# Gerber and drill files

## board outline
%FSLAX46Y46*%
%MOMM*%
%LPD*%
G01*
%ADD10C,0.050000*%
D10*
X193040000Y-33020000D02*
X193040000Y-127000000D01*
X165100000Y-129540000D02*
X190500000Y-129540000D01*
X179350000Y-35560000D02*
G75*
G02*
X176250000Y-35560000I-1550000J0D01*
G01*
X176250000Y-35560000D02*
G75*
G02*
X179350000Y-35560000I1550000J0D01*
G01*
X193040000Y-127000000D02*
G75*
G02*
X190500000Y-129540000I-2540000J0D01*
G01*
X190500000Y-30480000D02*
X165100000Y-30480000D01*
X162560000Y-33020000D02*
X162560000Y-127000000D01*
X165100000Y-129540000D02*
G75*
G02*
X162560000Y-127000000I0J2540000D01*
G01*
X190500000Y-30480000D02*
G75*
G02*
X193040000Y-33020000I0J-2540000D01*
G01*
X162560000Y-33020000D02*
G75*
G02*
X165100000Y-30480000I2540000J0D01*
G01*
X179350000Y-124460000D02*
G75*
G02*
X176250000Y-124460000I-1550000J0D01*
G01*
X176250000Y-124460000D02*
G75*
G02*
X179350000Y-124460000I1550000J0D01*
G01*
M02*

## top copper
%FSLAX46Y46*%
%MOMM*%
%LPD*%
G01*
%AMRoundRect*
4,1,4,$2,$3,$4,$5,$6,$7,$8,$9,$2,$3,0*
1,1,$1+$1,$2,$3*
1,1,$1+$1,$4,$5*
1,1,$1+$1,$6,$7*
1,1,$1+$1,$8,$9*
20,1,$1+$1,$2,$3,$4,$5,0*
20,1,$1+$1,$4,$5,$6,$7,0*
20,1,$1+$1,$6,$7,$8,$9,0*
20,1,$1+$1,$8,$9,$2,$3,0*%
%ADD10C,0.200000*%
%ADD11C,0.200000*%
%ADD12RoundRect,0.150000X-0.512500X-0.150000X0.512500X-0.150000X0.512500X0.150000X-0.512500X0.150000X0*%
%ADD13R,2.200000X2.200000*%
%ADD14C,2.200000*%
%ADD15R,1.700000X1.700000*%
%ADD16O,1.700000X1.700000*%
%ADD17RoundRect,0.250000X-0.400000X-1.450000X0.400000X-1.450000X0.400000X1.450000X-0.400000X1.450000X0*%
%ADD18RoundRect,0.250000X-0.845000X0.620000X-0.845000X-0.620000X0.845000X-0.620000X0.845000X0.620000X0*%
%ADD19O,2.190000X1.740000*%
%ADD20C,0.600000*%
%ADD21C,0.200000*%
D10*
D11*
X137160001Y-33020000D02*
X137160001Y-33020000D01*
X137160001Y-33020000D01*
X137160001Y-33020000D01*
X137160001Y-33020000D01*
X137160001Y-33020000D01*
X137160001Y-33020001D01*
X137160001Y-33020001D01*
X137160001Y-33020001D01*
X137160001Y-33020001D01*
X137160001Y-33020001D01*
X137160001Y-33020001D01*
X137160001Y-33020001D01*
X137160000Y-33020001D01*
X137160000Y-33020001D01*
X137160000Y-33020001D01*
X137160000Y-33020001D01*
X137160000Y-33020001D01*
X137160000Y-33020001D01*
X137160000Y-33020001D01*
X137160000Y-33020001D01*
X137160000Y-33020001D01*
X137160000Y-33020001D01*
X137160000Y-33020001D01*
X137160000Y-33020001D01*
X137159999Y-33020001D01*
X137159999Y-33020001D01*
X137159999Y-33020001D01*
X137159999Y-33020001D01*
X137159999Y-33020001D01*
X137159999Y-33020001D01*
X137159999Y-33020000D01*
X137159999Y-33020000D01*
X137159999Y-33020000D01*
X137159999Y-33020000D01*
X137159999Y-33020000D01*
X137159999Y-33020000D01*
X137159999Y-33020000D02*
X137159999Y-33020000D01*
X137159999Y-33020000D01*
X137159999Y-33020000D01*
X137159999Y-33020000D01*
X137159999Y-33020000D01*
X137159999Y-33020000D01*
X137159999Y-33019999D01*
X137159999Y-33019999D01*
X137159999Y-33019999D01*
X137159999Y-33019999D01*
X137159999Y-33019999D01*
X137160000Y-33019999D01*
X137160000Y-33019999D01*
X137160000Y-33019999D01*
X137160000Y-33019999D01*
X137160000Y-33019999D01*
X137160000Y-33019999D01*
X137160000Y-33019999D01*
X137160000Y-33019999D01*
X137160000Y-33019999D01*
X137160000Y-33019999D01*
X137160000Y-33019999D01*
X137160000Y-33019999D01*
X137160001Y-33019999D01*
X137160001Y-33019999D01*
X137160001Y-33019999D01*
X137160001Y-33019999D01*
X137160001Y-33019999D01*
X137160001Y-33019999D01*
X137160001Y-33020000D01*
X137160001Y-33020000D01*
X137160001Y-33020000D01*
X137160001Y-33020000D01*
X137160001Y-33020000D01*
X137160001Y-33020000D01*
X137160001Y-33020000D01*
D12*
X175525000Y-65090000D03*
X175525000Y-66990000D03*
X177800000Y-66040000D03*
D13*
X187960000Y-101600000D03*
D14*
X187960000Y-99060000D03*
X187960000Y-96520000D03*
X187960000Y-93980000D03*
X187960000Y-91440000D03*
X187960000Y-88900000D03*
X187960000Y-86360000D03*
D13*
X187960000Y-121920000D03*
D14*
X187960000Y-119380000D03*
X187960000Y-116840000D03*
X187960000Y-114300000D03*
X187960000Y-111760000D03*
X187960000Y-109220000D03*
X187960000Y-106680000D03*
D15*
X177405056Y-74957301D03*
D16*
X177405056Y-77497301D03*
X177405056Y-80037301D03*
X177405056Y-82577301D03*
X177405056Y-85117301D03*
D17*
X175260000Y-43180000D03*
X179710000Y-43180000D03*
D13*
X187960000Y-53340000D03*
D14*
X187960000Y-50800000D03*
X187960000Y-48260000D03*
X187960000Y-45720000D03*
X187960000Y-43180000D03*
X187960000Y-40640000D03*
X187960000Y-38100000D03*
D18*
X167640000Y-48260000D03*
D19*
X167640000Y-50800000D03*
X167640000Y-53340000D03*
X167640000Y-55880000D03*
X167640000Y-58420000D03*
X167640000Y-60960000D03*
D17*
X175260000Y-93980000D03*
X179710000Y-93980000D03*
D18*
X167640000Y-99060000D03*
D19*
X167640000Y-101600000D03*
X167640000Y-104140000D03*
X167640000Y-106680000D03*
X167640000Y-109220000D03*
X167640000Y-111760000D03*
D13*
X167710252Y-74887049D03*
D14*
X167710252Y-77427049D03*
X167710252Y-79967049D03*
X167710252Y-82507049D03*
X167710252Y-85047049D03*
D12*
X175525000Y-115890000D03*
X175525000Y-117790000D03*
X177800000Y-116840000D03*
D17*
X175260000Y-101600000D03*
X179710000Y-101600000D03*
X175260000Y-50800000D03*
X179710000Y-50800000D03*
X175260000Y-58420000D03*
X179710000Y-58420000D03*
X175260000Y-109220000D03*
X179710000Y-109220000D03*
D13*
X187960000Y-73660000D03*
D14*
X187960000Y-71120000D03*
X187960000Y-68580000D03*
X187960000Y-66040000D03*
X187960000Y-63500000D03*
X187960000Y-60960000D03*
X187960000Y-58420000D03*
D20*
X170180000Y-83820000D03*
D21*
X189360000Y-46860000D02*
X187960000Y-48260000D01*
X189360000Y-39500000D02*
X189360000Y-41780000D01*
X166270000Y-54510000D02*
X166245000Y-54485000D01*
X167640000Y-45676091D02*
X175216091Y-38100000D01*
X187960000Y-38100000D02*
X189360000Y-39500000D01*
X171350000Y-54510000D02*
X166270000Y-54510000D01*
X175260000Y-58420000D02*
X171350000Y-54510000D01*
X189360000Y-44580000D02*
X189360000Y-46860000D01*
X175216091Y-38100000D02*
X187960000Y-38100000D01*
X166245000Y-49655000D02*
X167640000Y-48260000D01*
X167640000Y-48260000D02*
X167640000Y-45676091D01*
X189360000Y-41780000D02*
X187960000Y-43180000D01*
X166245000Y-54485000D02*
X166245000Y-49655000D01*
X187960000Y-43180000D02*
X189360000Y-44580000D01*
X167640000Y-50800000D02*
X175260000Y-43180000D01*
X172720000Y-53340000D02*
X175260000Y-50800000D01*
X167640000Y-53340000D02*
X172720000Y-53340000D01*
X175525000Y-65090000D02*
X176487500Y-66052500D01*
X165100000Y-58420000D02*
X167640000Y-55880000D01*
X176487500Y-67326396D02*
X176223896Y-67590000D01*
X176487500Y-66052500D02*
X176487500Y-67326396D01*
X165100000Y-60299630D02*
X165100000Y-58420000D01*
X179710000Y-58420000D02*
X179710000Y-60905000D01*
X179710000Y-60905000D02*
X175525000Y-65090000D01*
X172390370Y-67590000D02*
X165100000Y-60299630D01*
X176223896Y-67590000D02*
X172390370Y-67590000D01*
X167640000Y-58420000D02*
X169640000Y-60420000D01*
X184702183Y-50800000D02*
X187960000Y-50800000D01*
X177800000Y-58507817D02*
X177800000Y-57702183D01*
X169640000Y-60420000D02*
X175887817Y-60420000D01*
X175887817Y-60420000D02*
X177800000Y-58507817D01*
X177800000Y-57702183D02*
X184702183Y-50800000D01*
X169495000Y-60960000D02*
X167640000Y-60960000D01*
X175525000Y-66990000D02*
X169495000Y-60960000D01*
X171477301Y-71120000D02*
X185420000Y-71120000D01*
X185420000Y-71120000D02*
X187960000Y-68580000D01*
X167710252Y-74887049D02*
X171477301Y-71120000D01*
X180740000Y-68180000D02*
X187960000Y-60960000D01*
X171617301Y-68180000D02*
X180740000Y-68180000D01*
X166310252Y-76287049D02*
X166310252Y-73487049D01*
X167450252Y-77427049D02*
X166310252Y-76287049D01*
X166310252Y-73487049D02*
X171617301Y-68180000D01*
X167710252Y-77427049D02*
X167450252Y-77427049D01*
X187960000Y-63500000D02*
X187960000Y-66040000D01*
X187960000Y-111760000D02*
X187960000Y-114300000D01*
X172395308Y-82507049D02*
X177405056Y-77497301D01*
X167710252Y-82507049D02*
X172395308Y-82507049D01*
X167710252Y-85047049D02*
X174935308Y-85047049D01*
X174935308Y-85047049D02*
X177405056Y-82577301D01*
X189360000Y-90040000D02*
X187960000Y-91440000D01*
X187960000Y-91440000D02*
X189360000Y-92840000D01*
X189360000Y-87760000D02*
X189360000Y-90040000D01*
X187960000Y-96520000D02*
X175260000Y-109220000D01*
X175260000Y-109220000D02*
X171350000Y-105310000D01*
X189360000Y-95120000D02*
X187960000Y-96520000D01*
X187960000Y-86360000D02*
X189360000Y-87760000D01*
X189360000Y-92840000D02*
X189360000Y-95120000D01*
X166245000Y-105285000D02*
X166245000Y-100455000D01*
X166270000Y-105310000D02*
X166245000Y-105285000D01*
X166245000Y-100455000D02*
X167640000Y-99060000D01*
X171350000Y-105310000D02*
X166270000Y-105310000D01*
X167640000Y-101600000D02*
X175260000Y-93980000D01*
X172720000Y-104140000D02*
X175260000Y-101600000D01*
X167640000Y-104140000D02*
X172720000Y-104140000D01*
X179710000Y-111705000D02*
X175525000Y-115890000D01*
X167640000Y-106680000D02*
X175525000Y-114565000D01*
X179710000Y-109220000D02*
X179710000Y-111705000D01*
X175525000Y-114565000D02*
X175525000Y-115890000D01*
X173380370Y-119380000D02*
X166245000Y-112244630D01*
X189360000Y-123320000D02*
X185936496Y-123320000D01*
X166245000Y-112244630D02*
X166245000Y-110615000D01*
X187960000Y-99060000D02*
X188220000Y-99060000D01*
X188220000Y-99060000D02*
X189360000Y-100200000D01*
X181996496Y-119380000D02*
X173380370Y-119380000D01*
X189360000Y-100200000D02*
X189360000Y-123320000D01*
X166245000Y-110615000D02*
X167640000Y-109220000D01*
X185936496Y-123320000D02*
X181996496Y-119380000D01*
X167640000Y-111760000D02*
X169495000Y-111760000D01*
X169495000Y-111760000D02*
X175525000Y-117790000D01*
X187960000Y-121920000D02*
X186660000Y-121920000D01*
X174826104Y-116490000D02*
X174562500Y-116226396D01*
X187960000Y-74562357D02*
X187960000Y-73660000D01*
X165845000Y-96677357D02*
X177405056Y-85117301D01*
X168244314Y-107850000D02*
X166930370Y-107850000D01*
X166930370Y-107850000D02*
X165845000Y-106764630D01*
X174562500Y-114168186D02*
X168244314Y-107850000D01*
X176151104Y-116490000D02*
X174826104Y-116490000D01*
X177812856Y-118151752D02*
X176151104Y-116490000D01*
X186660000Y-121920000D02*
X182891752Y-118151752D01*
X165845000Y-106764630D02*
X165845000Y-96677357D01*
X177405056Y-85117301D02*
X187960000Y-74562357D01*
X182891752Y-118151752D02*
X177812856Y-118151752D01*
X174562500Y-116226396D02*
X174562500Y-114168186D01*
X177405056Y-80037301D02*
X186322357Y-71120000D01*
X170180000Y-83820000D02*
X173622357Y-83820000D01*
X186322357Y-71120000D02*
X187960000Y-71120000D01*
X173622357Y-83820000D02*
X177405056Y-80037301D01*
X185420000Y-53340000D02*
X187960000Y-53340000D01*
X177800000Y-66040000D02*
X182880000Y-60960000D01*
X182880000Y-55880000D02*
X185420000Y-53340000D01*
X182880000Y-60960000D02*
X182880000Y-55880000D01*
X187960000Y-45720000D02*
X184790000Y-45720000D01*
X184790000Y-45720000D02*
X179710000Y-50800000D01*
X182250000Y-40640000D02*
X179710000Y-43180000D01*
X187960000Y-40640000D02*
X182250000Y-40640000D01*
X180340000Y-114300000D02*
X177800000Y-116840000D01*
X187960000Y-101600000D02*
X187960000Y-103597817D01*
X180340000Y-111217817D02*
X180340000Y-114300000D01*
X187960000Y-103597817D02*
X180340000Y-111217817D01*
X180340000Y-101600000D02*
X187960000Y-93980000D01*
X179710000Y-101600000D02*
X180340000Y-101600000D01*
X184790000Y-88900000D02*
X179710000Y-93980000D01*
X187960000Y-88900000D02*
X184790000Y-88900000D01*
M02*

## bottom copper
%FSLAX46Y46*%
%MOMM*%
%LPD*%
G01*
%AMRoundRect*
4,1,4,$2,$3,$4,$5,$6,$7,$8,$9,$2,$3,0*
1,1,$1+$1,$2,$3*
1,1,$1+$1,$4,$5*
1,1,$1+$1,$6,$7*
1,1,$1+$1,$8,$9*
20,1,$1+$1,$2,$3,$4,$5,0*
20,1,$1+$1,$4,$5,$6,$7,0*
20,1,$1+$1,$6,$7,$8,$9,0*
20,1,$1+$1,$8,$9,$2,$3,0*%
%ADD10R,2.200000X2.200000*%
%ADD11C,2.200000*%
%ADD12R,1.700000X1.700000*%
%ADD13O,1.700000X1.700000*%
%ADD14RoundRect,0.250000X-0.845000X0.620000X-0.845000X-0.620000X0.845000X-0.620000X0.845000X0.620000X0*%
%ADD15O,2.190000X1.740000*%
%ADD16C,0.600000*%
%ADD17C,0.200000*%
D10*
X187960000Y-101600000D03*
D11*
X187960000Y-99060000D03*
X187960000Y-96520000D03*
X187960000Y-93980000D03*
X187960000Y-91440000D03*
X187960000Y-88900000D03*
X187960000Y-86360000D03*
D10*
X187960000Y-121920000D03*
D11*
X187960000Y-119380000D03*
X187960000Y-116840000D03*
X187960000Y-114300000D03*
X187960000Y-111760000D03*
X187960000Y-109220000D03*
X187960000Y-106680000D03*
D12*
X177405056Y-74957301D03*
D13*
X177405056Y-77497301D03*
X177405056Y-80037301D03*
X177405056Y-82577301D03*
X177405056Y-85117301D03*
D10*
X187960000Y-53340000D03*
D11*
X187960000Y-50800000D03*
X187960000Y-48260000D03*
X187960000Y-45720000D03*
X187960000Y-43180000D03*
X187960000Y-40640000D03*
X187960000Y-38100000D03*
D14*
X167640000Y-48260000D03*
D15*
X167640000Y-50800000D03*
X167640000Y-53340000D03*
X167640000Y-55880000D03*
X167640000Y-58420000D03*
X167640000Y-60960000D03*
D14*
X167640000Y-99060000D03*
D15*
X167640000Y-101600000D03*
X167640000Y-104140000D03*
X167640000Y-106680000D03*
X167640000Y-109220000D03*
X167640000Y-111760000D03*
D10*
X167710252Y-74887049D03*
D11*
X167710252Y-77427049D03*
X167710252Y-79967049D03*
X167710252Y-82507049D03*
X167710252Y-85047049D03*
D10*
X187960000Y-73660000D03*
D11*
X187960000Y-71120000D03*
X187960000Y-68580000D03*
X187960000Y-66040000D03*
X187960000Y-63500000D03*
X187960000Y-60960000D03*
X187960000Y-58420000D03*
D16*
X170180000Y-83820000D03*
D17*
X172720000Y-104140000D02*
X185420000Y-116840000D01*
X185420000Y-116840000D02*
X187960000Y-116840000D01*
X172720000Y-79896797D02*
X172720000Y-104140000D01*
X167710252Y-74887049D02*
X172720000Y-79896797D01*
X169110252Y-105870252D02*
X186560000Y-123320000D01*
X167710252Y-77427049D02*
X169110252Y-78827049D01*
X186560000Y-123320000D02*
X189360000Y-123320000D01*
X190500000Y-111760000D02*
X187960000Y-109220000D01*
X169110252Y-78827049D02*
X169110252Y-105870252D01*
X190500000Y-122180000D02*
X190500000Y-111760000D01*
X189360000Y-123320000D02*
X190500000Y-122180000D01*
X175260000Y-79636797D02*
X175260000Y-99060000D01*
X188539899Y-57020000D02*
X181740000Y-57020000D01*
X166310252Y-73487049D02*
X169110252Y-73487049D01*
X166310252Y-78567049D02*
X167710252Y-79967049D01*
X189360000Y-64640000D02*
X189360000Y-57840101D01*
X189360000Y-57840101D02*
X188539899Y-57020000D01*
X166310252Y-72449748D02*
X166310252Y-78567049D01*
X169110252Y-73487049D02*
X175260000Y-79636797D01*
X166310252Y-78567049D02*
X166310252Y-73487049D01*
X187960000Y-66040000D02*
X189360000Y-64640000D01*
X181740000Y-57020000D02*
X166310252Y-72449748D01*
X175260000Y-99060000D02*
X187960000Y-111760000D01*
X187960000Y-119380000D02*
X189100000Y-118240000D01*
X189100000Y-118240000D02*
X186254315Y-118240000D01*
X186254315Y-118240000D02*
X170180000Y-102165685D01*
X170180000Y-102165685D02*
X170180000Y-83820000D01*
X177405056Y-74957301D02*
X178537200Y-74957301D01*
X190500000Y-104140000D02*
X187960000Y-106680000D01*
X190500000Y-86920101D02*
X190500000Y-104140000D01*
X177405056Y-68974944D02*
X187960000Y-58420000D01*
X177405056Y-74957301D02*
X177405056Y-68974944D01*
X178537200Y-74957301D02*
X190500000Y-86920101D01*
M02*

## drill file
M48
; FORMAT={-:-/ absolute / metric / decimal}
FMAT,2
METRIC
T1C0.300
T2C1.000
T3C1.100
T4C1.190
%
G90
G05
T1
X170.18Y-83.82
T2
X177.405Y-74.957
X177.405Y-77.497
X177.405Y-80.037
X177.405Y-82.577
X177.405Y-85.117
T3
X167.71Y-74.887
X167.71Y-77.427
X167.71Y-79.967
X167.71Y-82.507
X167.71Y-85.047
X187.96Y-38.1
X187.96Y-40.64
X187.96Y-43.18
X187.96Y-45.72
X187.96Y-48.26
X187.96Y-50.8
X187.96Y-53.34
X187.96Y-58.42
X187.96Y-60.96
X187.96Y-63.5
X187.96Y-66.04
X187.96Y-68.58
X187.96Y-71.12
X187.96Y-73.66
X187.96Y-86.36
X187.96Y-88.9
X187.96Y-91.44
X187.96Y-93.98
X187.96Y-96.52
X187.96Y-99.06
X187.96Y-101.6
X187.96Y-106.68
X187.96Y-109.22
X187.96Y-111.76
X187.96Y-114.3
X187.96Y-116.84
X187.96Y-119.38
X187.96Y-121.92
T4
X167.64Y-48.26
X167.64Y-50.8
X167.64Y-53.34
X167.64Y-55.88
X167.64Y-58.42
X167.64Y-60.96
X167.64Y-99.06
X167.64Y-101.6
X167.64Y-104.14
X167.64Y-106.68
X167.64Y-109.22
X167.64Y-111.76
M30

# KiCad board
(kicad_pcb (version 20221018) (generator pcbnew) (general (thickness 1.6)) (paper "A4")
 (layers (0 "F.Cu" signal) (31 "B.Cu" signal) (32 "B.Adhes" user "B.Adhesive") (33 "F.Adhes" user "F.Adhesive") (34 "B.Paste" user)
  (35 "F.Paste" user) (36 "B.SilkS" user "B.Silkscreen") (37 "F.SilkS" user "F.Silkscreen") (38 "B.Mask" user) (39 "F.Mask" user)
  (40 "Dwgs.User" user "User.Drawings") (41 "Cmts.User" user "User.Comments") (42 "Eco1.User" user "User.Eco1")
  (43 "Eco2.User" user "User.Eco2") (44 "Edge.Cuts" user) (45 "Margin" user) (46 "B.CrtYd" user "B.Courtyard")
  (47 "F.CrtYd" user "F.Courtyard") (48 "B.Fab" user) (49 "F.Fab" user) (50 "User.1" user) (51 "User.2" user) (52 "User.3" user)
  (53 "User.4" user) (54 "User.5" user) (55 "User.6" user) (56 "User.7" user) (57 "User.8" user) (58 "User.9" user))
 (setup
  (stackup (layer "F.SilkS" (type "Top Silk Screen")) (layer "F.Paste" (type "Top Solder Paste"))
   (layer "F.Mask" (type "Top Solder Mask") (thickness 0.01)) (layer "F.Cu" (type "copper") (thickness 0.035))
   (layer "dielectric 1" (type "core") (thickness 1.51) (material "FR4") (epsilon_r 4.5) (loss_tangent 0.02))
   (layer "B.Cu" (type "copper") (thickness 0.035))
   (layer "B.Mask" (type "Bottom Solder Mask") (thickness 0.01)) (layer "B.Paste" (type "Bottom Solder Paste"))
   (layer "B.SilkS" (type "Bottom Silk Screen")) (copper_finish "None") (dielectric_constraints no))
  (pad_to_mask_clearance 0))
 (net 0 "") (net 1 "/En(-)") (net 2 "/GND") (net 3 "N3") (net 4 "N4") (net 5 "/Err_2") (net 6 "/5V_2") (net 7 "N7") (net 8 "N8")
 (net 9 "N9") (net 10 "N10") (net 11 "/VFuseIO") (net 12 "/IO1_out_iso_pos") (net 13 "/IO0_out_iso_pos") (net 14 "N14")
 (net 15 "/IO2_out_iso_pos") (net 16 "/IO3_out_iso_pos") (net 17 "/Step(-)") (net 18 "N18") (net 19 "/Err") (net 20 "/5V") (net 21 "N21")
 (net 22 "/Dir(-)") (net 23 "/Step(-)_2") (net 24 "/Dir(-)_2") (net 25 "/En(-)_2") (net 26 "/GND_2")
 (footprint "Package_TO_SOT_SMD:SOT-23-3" (layer "F.Cu") (at 176.6625 66.04)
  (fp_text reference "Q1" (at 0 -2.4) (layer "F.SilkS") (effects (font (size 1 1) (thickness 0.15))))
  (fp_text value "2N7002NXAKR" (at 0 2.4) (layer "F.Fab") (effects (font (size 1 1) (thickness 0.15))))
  (pad "1" smd roundrect (at -1.1375 -0.95) (size 1.325 0.6) (layers "F.Cu" "F.Paste" "F.Mask") (roundrect_rratio 0.25) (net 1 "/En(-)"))
  (pad "2" smd roundrect (at -1.1375 0.95) (size 1.325 0.6) (layers "F.Cu" "F.Paste" "F.Mask") (roundrect_rratio 0.25) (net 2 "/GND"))
  (pad "3" smd roundrect (at 1.1375 0) (size 1.325 0.6) (layers "F.Cu" "F.Paste" "F.Mask") (roundrect_rratio 0.25) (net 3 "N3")))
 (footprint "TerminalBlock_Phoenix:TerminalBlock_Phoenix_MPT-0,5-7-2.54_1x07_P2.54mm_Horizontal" (layer "F.Cu") (at 187.96 101.6 90)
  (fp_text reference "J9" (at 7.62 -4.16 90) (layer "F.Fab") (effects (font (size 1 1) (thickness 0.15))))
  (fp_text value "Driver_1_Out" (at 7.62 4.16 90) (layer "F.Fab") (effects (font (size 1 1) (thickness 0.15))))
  (pad "1" thru_hole rect (at 0 0 90) (size 2.2 2.2) (drill 1.1) (layers "*.Cu" "*.Mask") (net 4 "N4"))
  (pad "2" thru_hole circle (at 2.54 0 90) (size 2.2 2.2) (drill 1.1) (layers "*.Cu" "*.Mask") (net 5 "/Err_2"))
  (pad "3" thru_hole circle (at 5.08 0 90) (size 2.2 2.2) (drill 1.1) (layers "*.Cu" "*.Mask") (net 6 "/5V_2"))
  (pad "4" thru_hole circle (at 7.62 0 90) (size 2.2 2.2) (drill 1.1) (layers "*.Cu" "*.Mask") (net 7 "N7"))
  (pad "5" thru_hole circle (at 10.16 0 90) (size 2.2 2.2) (drill 1.1) (layers "*.Cu" "*.Mask") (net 6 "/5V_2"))
  (pad "6" thru_hole circle (at 12.7 0 90) (size 2.2 2.2) (drill 1.1) (layers "*.Cu" "*.Mask") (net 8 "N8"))
  (pad "7" thru_hole circle (at 15.24 0 90) (size 2.2 2.2) (drill 1.1) (layers "*.Cu" "*.Mask") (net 6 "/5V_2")))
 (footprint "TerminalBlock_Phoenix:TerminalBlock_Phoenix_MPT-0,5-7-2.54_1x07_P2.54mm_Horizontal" (layer "F.Cu") (at 187.96 121.92 90)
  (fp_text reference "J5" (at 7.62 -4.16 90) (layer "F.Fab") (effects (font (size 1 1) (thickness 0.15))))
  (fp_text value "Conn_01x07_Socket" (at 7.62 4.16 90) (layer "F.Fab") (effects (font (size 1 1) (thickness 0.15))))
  (pad "1" thru_hole rect (at 0 0 90) (size 2.2 2.2) (drill 1.1) (layers "*.Cu" "*.Mask") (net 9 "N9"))
  (pad "2" thru_hole circle (at 2.54 0 90) (size 2.2 2.2) (drill 1.1) (layers "*.Cu" "*.Mask") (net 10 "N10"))
  (pad "3" thru_hole circle (at 5.08 0 90) (size 2.2 2.2) (drill 1.1) (layers "*.Cu" "*.Mask") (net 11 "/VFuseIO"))
  (pad "4" thru_hole circle (at 7.62 0 90) (size 2.2 2.2) (drill 1.1) (layers "*.Cu" "*.Mask") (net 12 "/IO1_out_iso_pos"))
  (pad "5" thru_hole circle (at 10.16 0 90) (size 2.2 2.2) (drill 1.1) (layers "*.Cu" "*.Mask") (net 12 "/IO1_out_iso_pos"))
  (pad "6" thru_hole circle (at 12.7 0 90) (size 2.2 2.2) (drill 1.1) (layers "*.Cu" "*.Mask") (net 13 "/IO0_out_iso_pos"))
  (pad "7" thru_hole circle (at 15.24 0 90) (size 2.2 2.2) (drill 1.1) (layers "*.Cu" "*.Mask") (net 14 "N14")))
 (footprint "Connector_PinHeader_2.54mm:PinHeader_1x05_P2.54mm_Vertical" (layer "F.Cu") (at 177.405056 74.957301)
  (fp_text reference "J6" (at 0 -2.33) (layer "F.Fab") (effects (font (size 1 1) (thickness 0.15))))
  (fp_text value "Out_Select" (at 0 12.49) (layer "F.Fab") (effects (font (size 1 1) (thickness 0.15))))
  (pad "1" thru_hole rect (at 0 0) (size 1.7 1.7) (drill 1) (layers "*.Cu" "*.Mask") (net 14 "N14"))
  (pad "2" thru_hole oval (at 0 2.54) (size 1.7 1.7) (drill 1) (layers "*.Cu" "*.Mask") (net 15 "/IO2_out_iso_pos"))
  (pad "3" thru_hole oval (at 0 5.08) (size 1.7 1.7) (drill 1) (layers "*.Cu" "*.Mask") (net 10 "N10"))
  (pad "4" thru_hole oval (at 0 7.62) (size 1.7 1.7) (drill 1) (layers "*.Cu" "*.Mask") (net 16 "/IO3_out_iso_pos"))
  (pad "5" thru_hole oval (at 0 10.16) (size 1.7 1.7) (drill 1) (layers "*.Cu" "*.Mask") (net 9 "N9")))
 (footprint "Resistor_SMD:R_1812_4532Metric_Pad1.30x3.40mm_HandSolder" (layer "F.Cu") (at 177.485 43.18)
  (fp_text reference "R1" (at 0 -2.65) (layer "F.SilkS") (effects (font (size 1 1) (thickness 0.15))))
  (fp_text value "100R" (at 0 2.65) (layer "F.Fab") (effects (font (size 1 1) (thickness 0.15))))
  (pad "1" smd roundrect (at -2.225 0) (size 1.3 3.4) (layers "F.Cu" "F.Paste" "F.Mask") (roundrect_rratio 0.1923076923) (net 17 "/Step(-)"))
  (pad "2" smd roundrect (at 2.225 0) (size 1.3 3.4) (layers "F.Cu" "F.Paste" "F.Mask") (roundrect_rratio 0.1923076923) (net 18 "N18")))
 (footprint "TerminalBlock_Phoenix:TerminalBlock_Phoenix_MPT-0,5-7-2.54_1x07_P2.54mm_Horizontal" (layer "F.Cu") (at 187.96 53.34 90)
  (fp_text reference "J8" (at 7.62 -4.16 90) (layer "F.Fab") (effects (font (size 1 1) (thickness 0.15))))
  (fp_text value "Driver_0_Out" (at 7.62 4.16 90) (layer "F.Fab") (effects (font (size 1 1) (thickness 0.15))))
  (pad "1" thru_hole rect (at 0 0 90) (size 2.2 2.2) (drill 1.1) (layers "*.Cu" "*.Mask") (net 3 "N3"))
  (pad "2" thru_hole circle (at 2.54 0 90) (size 2.2 2.2) (drill 1.1) (layers "*.Cu" "*.Mask") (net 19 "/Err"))
  (pad "3" thru_hole circle (at 5.08 0 90) (size 2.2 2.2) (drill 1.1) (layers "*.Cu" "*.Mask") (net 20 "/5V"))
  (pad "4" thru_hole circle (at 7.62 0 90) (size 2.2 2.2) (drill 1.1) (layers "*.Cu" "*.Mask") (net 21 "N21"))
  (pad "5" thru_hole circle (at 10.16 0 90) (size 2.2 2.2) (drill 1.1) (layers "*.Cu" "*.Mask") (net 20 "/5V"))
  (pad "6" thru_hole circle (at 12.7 0 90) (size 2.2 2.2) (drill 1.1) (layers "*.Cu" "*.Mask") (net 18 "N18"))
  (pad "7" thru_hole circle (at 15.24 0 90) (size 2.2 2.2) (drill 1.1) (layers "*.Cu" "*.Mask") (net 20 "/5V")))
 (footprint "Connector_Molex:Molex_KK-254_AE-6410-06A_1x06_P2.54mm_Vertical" (layer "F.Cu") (at 167.64 48.26 -90)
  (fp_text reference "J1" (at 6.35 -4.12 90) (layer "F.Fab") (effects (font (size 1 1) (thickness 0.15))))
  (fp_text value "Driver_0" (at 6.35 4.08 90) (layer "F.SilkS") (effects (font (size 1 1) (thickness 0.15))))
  (pad "1" thru_hole roundrect (at 0 0 270) (size 1.74 2.19) (drill 1.19) (layers "*.Cu" "*.Mask") (roundrect_rratio 0.1436781609)
   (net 20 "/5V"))
  (pad "2" thru_hole oval (at 2.54 0 270) (size 1.74 2.19) (drill 1.19) (layers "*.Cu" "*.Mask") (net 17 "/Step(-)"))
  (pad "3" thru_hole oval (at 5.08 0 270) (size 1.74 2.19) (drill 1.19) (layers "*.Cu" "*.Mask") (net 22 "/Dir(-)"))
  (pad "4" thru_hole oval (at 7.62 0 270) (size 1.74 2.19) (drill 1.19) (layers "*.Cu" "*.Mask") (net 1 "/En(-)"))
  (pad "5" thru_hole oval (at 10.16 0 270) (size 1.74 2.19) (drill 1.19) (layers "*.Cu" "*.Mask") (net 19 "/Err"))
  (pad "6" thru_hole oval (at 12.7 0 270) (size 1.74 2.19) (drill 1.19) (layers "*.Cu" "*.Mask") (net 2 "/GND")))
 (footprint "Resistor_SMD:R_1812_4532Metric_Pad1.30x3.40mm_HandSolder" (layer "F.Cu") (at 177.485 93.98)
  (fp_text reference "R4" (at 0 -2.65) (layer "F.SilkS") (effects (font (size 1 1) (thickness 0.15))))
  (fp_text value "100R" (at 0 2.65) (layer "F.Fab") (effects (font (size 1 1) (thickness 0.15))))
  (pad "1" smd roundrect (at -2.225 0) (size 1.3 3.4) (layers "F.Cu" "F.Paste" "F.Mask") (roundrect_rratio 0.1923076923)
   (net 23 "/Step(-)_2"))
  (pad "2" smd roundrect (at 2.225 0) (size 1.3 3.4) (layers "F.Cu" "F.Paste" "F.Mask") (roundrect_rratio 0.1923076923) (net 8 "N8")))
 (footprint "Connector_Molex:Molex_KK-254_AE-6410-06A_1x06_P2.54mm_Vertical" (layer "F.Cu") (at 167.64 99.06 -90)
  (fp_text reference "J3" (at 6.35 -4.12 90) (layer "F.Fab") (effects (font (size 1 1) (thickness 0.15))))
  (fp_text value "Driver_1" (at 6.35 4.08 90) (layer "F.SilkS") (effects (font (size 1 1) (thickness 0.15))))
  (pad "1" thru_hole roundrect (at 0 0 270) (size 1.74 2.19) (drill 1.19) (layers "*.Cu" "*.Mask") (roundrect_rratio 0.1436781609)
   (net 6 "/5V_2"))
  (pad "2" thru_hole oval (at 2.54 0 270) (size 1.74 2.19) (drill 1.19) (layers "*.Cu" "*.Mask") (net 23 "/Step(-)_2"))
  (pad "3" thru_hole oval (at 5.08 0 270) (size 1.74 2.19) (drill 1.19) (layers "*.Cu" "*.Mask") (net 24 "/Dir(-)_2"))
  (pad "4" thru_hole oval (at 7.62 0 270) (size 1.74 2.19) (drill 1.19) (layers "*.Cu" "*.Mask") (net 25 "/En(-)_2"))
  (pad "5" thru_hole oval (at 10.16 0 270) (size 1.74 2.19) (drill 1.19) (layers "*.Cu" "*.Mask") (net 5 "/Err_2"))
  (pad "6" thru_hole oval (at 12.7 0 270) (size 1.74 2.19) (drill 1.19) (layers "*.Cu" "*.Mask") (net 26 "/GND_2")))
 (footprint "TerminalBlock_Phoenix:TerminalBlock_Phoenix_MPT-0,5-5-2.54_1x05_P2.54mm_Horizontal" (layer "F.Cu")
  (at 167.710252 74.887049 -90)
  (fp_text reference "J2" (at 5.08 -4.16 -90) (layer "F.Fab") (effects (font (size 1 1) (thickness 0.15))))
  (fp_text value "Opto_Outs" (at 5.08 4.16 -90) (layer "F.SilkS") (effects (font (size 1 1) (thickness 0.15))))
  (pad "1" thru_hole rect (at 0 0 270) (size 2.2 2.2) (drill 1.1) (layers "*.Cu" "*.Mask") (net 11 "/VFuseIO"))
  (pad "2" thru_hole circle (at 2.54 0 270) (size 2.2 2.2) (drill 1.1) (layers "*.Cu" "*.Mask") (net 13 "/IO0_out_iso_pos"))
  (pad "3" thru_hole circle (at 5.08 0 270) (size 2.2 2.2) (drill 1.1) (layers "*.Cu" "*.Mask") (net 12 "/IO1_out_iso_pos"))
  (pad "4" thru_hole circle (at 7.62 0 270) (size 2.2 2.2) (drill 1.1) (layers "*.Cu" "*.Mask") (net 15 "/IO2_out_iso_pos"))
  (pad "5" thru_hole circle (at 10.16 0 270) (size 2.2 2.2) (drill 1.1) (layers "*.Cu" "*.Mask") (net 16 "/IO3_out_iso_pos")))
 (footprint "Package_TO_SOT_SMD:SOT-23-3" (layer "F.Cu") (at 176.6625 116.84)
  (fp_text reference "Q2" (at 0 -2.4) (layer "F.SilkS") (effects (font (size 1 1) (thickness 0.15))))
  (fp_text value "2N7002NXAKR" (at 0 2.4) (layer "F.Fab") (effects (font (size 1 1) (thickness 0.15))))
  (pad "1" smd roundrect (at -1.1375 -0.95) (size 1.325 0.6) (layers "F.Cu" "F.Paste" "F.Mask") (roundrect_rratio 0.25) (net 25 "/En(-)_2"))
  (pad "2" smd roundrect (at -1.1375 0.95) (size 1.325 0.6) (layers "F.Cu" "F.Paste" "F.Mask") (roundrect_rratio 0.25) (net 26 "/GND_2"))
  (pad "3" smd roundrect (at 1.1375 0) (size 1.325 0.6) (layers "F.Cu" "F.Paste" "F.Mask") (roundrect_rratio 0.25) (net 4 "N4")))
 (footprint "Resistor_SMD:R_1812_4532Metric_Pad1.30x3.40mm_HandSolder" (layer "F.Cu") (at 177.485 101.6)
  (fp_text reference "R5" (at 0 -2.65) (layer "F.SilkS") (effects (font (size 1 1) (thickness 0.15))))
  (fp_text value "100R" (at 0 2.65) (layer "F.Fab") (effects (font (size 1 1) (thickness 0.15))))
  (pad "1" smd roundrect (at -2.225 0) (size 1.3 3.4) (layers "F.Cu" "F.Paste" "F.Mask") (roundrect_rratio 0.1923076923)
   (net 24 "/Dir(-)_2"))
  (pad "2" smd roundrect (at 2.225 0) (size 1.3 3.4) (layers "F.Cu" "F.Paste" "F.Mask") (roundrect_rratio 0.1923076923) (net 7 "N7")))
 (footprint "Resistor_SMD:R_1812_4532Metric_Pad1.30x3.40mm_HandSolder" (layer "F.Cu") (at 177.485 50.8)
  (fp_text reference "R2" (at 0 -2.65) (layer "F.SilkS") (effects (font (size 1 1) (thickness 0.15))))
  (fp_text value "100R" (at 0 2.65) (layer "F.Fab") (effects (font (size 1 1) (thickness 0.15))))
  (pad "1" smd roundrect (at -2.225 0) (size 1.3 3.4) (layers "F.Cu" "F.Paste" "F.Mask") (roundrect_rratio 0.1923076923) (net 22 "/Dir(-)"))
  (pad "2" smd roundrect (at 2.225 0) (size 1.3 3.4) (layers "F.Cu" "F.Paste" "F.Mask") (roundrect_rratio 0.1923076923) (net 21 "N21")))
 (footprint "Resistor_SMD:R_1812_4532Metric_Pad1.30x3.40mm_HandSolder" (layer "F.Cu") (at 177.485 58.42)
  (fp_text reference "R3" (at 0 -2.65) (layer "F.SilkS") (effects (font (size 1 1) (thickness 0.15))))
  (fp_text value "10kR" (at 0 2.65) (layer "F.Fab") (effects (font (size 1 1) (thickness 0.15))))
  (pad "1" smd roundrect (at -2.225 0) (size 1.3 3.4) (layers "F.Cu" "F.Paste" "F.Mask") (roundrect_rratio 0.1923076923) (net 20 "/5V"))
  (pad "2" smd roundrect (at 2.225 0) (size 1.3 3.4) (layers "F.Cu" "F.Paste" "F.Mask") (roundrect_rratio 0.1923076923) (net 1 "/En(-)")))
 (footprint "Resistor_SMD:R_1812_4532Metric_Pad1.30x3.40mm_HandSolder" (layer "F.Cu") (at 177.485 109.22)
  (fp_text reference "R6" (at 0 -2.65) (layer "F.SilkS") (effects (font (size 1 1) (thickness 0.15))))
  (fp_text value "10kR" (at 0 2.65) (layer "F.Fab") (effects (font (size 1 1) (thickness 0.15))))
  (pad "1" smd roundrect (at -2.225 0) (size 1.3 3.4) (layers "F.Cu" "F.Paste" "F.Mask") (roundrect_rratio 0.1923076923) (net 6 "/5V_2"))
  (pad "2" smd roundrect (at 2.225 0) (size 1.3 3.4) (layers "F.Cu" "F.Paste" "F.Mask") (roundrect_rratio 0.1923076923) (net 25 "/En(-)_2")))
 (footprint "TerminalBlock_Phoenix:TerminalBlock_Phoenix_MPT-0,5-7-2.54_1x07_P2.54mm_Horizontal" (layer "F.Cu") (at 187.96 73.66 90)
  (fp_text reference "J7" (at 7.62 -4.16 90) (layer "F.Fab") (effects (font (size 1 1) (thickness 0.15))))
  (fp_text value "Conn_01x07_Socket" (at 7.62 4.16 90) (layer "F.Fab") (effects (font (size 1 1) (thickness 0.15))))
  (pad "1" thru_hole rect (at 0 0 90) (size 2.2 2.2) (drill 1.1) (layers "*.Cu" "*.Mask") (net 9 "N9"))
  (pad "2" thru_hole circle (at 2.54 0 90) (size 2.2 2.2) (drill 1.1) (layers "*.Cu" "*.Mask") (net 10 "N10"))
  (pad "3" thru_hole circle (at 5.08 0 90) (size 2.2 2.2) (drill 1.1) (layers "*.Cu" "*.Mask") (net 11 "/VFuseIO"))
  (pad "4" thru_hole circle (at 7.62 0 90) (size 2.2 2.2) (drill 1.1) (layers "*.Cu" "*.Mask") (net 12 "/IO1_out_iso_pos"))
  (pad "5" thru_hole circle (at 10.16 0 90) (size 2.2 2.2) (drill 1.1) (layers "*.Cu" "*.Mask") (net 12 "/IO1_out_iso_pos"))
  (pad "6" thru_hole circle (at 12.7 0 90) (size 2.2 2.2) (drill 1.1) (layers "*.Cu" "*.Mask") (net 13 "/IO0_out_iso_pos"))
  (pad "7" thru_hole circle (at 15.24 0 90) (size 2.2 2.2) (drill 1.1) (layers "*.Cu" "*.Mask") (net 14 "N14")))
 (gr_circle (center 137.16 33.02) (end 137.16 33.02) (stroke (width 0.2) (type default)) (fill none) (layer "F.Cu"))
 (gr_line (start 193.04 33.02) (end 193.04 127) (stroke (width 0.05) (type default)) (layer "Edge.Cuts"))
 (gr_line (start 165.1 129.54) (end 190.5 129.54) (stroke (width 0.05) (type default)) (layer "Edge.Cuts"))
 (gr_circle (center 177.8 35.56) (end 179.35 35.56) (stroke (width 0.05) (type default)) (fill none) (layer "Edge.Cuts"))
 (gr_arc (start 193.04 127) (mid 192.296051 128.796051) (end 190.5 129.54) (stroke (width 0.05) (type default)) (layer "Edge.Cuts"))
 (gr_line (start 190.5 30.48) (end 165.1 30.48) (stroke (width 0.05) (type default)) (layer "Edge.Cuts"))
 (gr_line (start 162.56 33.02) (end 162.56 127) (stroke (width 0.05) (type default)) (layer "Edge.Cuts"))
 (gr_arc (start 165.1 129.54) (mid 163.303949 128.796051) (end 162.56 127) (stroke (width 0.05) (type default)) (layer "Edge.Cuts"))
 (gr_arc (start 190.5 30.48) (mid 192.296051 31.223949) (end 193.04 33.02) (stroke (width 0.05) (type default)) (layer "Edge.Cuts"))
 (gr_arc (start 162.56 33.02) (mid 163.303949 31.223949) (end 165.1 30.48) (stroke (width 0.05) (type default)) (layer "Edge.Cuts"))
 (gr_circle (center 177.8 124.46) (end 179.35 124.46) (stroke (width 0.05) (type default)) (fill none) (layer "Edge.Cuts"))
 (segment (start 189.36 46.86) (end 187.96 48.26) (width 0.2) (layer "F.Cu") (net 20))
 (segment (start 189.36 39.5) (end 189.36 41.78) (width 0.2) (layer "F.Cu") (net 20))
 (segment (start 166.27 54.51) (end 166.245 54.485) (width 0.2) (layer "F.Cu") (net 20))
 (segment (start 167.64 45.676091) (end 175.216091 38.1) (width 0.2) (layer "F.Cu") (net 20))
 (segment (start 187.96 38.1) (end 189.36 39.5) (width 0.2) (layer "F.Cu") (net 20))
 (segment (start 171.35 54.51) (end 166.27 54.51) (width 0.2) (layer "F.Cu") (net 20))
 (segment (start 175.26 58.42) (end 171.35 54.51) (width 0.2) (layer "F.Cu") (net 20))
 (segment (start 189.36 44.58) (end 189.36 46.86) (width 0.2) (layer "F.Cu") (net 20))
 (segment (start 175.216091 38.1) (end 187.96 38.1) (width 0.2) (layer "F.Cu") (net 20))
 (segment (start 166.245 49.655) (end 167.64 48.26) (width 0.2) (layer "F.Cu") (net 20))
 (segment (start 167.64 48.26) (end 167.64 45.676091) (width 0.2) (layer "F.Cu") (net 20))
 (segment (start 189.36 41.78) (end 187.96 43.18) (width 0.2) (layer "F.Cu") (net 20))
 (segment (start 166.245 54.485) (end 166.245 49.655) (width 0.2) (layer "F.Cu") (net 20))
 (segment (start 187.96 43.18) (end 189.36 44.58) (width 0.2) (layer "F.Cu") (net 20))
 (segment (start 167.64 50.8) (end 175.26 43.18) (width 0.2) (layer "F.Cu") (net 17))
 (segment (start 172.72 53.34) (end 175.26 50.8) (width 0.2) (layer "F.Cu") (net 22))
 (segment (start 167.64 53.34) (end 172.72 53.34) (width 0.2) (layer "F.Cu") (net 22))
 (segment (start 175.525 65.09) (end 176.4875 66.0525) (width 0.2) (layer "F.Cu") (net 1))
 (segment (start 165.1 58.42) (end 167.64 55.88) (width 0.2) (layer "F.Cu") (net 1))
 (segment (start 176.4875 67.326396) (end 176.223896 67.59) (width 0.2) (layer "F.Cu") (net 1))
 (segment (start 176.4875 66.0525) (end 176.4875 67.326396) (width 0.2) (layer "F.Cu") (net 1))
 (segment (start 165.1 60.29963) (end 165.1 58.42) (width 0.2) (layer "F.Cu") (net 1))
 (segment (start 179.71 58.42) (end 179.71 60.905) (width 0.2) (layer "F.Cu") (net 1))
 (segment (start 179.71 60.905) (end 175.525 65.09) (width 0.2) (layer "F.Cu") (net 1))
 (segment (start 172.39037 67.59) (end 165.1 60.29963) (width 0.2) (layer "F.Cu") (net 1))
 (segment (start 176.223896 67.59) (end 172.39037 67.59) (width 0.2) (layer "F.Cu") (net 1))
 (segment (start 167.64 58.42) (end 169.64 60.42) (width 0.2) (layer "F.Cu") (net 19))
 (segment (start 184.702183 50.8) (end 187.96 50.8) (width 0.2) (layer "F.Cu") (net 19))
 (segment (start 177.8 58.507817) (end 177.8 57.702183) (width 0.2) (layer "F.Cu") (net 19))
 (segment (start 169.64 60.42) (end 175.887817 60.42) (width 0.2) (layer "F.Cu") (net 19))
 (segment (start 175.887817 60.42) (end 177.8 58.507817) (width 0.2) (layer "F.Cu") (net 19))
 (segment (start 177.8 57.702183) (end 184.702183 50.8) (width 0.2) (layer "F.Cu") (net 19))
 (segment (start 169.495 60.96) (end 167.64 60.96) (width 0.2) (layer "F.Cu") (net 2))
 (segment (start 175.525 66.99) (end 169.495 60.96) (width 0.2) (layer "F.Cu") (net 2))
 (segment (start 171.477301 71.12) (end 185.42 71.12) (width 0.2) (layer "F.Cu") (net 11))
 (segment (start 185.42 71.12) (end 187.96 68.58) (width 0.2) (layer "F.Cu") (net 11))
 (segment (start 167.710252 74.887049) (end 171.477301 71.12) (width 0.2) (layer "F.Cu") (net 11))
 (segment (start 172.72 104.14) (end 185.42 116.84) (width 0.2) (layer "B.Cu") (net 11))
 (segment (start 185.42 116.84) (end 187.96 116.84) (width 0.2) (layer "B.Cu") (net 11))
 (segment (start 172.72 79.896797) (end 172.72 104.14) (width 0.2) (layer "B.Cu") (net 11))
 (segment (start 167.710252 74.887049) (end 172.72 79.896797) (width 0.2) (layer "B.Cu") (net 11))
 (segment (start 180.74 68.18) (end 187.96 60.96) (width 0.2) (layer "F.Cu") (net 13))
 (segment (start 171.617301 68.18) (end 180.74 68.18) (width 0.2) (layer "F.Cu") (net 13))
 (segment (start 166.310252 76.287049) (end 166.310252 73.487049) (width 0.2) (layer "F.Cu") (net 13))
 (segment (start 167.450252 77.427049) (end 166.310252 76.287049) (width 0.2) (layer "F.Cu") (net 13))
 (segment (start 166.310252 73.487049) (end 171.617301 68.18) (width 0.2) (layer "F.Cu") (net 13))
 (segment (start 167.710252 77.427049) (end 167.450252 77.427049) (width 0.2) (layer "F.Cu") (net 13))
 (segment (start 169.110252 105.870252) (end 186.56 123.32) (width 0.2) (layer "B.Cu") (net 13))
 (segment (start 167.710252 77.427049) (end 169.110252 78.827049) (width 0.2) (layer "B.Cu") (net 13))
 (segment (start 186.56 123.32) (end 189.36 123.32) (width 0.2) (layer "B.Cu") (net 13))
 (segment (start 190.5 111.76) (end 187.96 109.22) (width 0.2) (layer "B.Cu") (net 13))
 (segment (start 169.110252 78.827049) (end 169.110252 105.870252) (width 0.2) (layer "B.Cu") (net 13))
 (segment (start 190.5 122.18) (end 190.5 111.76) (width 0.2) (layer "B.Cu") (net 13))
 (segment (start 189.36 123.32) (end 190.5 122.18) (width 0.2) (layer "B.Cu") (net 13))
 (segment (start 187.96 63.5) (end 187.96 66.04) (width 0.2) (layer "F.Cu") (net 12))
 (segment (start 187.96 111.76) (end 187.96 114.3) (width 0.2) (layer "F.Cu") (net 12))
 (segment (start 175.26 79.636797) (end 175.26 99.06) (width 0.2) (layer "B.Cu") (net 12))
 (segment (start 188.539899 57.02) (end 181.74 57.02) (width 0.2) (layer "B.Cu") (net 12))
 (segment (start 166.310252 73.487049) (end 169.110252 73.487049) (width 0.2) (layer "B.Cu") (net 12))
 (segment (start 166.310252 78.567049) (end 167.710252 79.967049) (width 0.2) (layer "B.Cu") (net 12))
 (segment (start 189.36 64.64) (end 189.36 57.840101) (width 0.2) (layer "B.Cu") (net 12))
 (segment (start 189.36 57.840101) (end 188.539899 57.02) (width 0.2) (layer "B.Cu") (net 12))
 (segment (start 166.310252 72.449748) (end 166.310252 78.567049) (width 0.2) (layer "B.Cu") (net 12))
 (segment (start 169.110252 73.487049) (end 175.26 79.636797) (width 0.2) (layer "B.Cu") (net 12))
 (segment (start 166.310252 78.567049) (end 166.310252 73.487049) (width 0.2) (layer "B.Cu") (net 12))
 (segment (start 187.96 66.04) (end 189.36 64.64) (width 0.2) (layer "B.Cu") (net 12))
 (segment (start 181.74 57.02) (end 166.310252 72.449748) (width 0.2) (layer "B.Cu") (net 12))
 (segment (start 175.26 99.06) (end 187.96 111.76) (width 0.2) (layer "B.Cu") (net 12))
 (segment (start 172.395308 82.507049) (end 177.405056 77.497301) (width 0.2) (layer "F.Cu") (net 15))
 (segment (start 167.710252 82.507049) (end 172.395308 82.507049) (width 0.2) (layer "F.Cu") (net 15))
 (segment (start 167.710252 85.047049) (end 174.935308 85.047049) (width 0.2) (layer "F.Cu") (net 16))
 (segment (start 174.935308 85.047049) (end 177.405056 82.577301) (width 0.2) (layer "F.Cu") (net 16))
 (segment (start 189.36 90.04) (end 187.96 91.44) (width 0.2) (layer "F.Cu") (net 6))
 (segment (start 187.96 91.44) (end 189.36 92.84) (width 0.2) (layer "F.Cu") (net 6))
 (segment (start 189.36 87.76) (end 189.36 90.04) (width 0.2) (layer "F.Cu") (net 6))
 (segment (start 187.96 96.52) (end 175.26 109.22) (width 0.2) (layer "F.Cu") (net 6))
 (segment (start 175.26 109.22) (end 171.35 105.31) (width 0.2) (layer "F.Cu") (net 6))
 (segment (start 189.36 95.12) (end 187.96 96.52) (width 0.2) (layer "F.Cu") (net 6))
 (segment (start 187.96 86.36) (end 189.36 87.76) (width 0.2) (layer "F.Cu") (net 6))
 (segment (start 189.36 92.84) (end 189.36 95.12) (width 0.2) (layer "F.Cu") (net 6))
 (segment (start 166.245 105.285) (end 166.245 100.455) (width 0.2) (layer "F.Cu") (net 6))
 (segment (start 166.27 105.31) (end 166.245 105.285) (width 0.2) (layer "F.Cu") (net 6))
 (segment (start 166.245 100.455) (end 167.64 99.06) (width 0.2) (layer "F.Cu") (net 6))
 (segment (start 171.35 105.31) (end 166.27 105.31) (width 0.2) (layer "F.Cu") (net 6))
 (segment (start 167.64 101.6) (end 175.26 93.98) (width 0.2) (layer "F.Cu") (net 23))
 (segment (start 172.72 104.14) (end 175.26 101.6) (width 0.2) (layer "F.Cu") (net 24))
 (segment (start 167.64 104.14) (end 172.72 104.14) (width 0.2) (layer "F.Cu") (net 24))
 (segment (start 179.71 111.705) (end 175.525 115.89) (width 0.2) (layer "F.Cu") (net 25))
 (segment (start 167.64 106.68) (end 175.525 114.565) (width 0.2) (layer "F.Cu") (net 25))
 (segment (start 179.71 109.22) (end 179.71 111.705) (width 0.2) (layer "F.Cu") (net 25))
 (segment (start 175.525 114.565) (end 175.525 115.89) (width 0.2) (layer "F.Cu") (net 25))
 (segment (start 173.38037 119.38) (end 166.245 112.24463) (width 0.2) (layer "F.Cu") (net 5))
 (segment (start 189.36 123.32) (end 185.936496 123.32) (width 0.2) (layer "F.Cu") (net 5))
 (segment (start 166.245 112.24463) (end 166.245 110.615) (width 0.2) (layer "F.Cu") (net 5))
 (segment (start 187.96 99.06) (end 188.22 99.06) (width 0.2) (layer "F.Cu") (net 5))
 (segment (start 188.22 99.06) (end 189.36 100.2) (width 0.2) (layer "F.Cu") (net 5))
 (segment (start 181.996496 119.38) (end 173.38037 119.38) (width 0.2) (layer "F.Cu") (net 5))
 (segment (start 189.36 100.2) (end 189.36 123.32) (width 0.2) (layer "F.Cu") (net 5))
 (segment (start 166.245 110.615) (end 167.64 109.22) (width 0.2) (layer "F.Cu") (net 5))
 (segment (start 185.936496 123.32) (end 181.996496 119.38) (width 0.2) (layer "F.Cu") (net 5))
 (segment (start 167.64 111.76) (end 169.495 111.76) (width 0.2) (layer "F.Cu") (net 26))
 (segment (start 169.495 111.76) (end 175.525 117.79) (width 0.2) (layer "F.Cu") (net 26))
 (segment (start 187.96 121.92) (end 186.66 121.92) (width 0.2) (layer "F.Cu") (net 9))
 (segment (start 174.826104 116.49) (end 174.5625 116.226396) (width 0.2) (layer "F.Cu") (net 9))
 (segment (start 187.96 74.562357) (end 187.96 73.66) (width 0.2) (layer "F.Cu") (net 9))
 (segment (start 165.845 96.677357) (end 177.405056 85.117301) (width 0.2) (layer "F.Cu") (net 9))
 (segment (start 168.244314 107.85) (end 166.93037 107.85) (width 0.2) (layer "F.Cu") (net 9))
 (segment (start 166.93037 107.85) (end 165.845 106.76463) (width 0.2) (layer "F.Cu") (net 9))
 (segment (start 174.5625 114.168186) (end 168.244314 107.85) (width 0.2) (layer "F.Cu") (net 9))
 (segment (start 176.151104 116.49) (end 174.826104 116.49) (width 0.2) (layer "F.Cu") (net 9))
 (segment (start 177.812856 118.151752) (end 176.151104 116.49) (width 0.2) (layer "F.Cu") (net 9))
 (segment (start 186.66 121.92) (end 182.891752 118.151752) (width 0.2) (layer "F.Cu") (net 9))
 (segment (start 165.845 106.76463) (end 165.845 96.677357) (width 0.2) (layer "F.Cu") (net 9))
 (segment (start 177.405056 85.117301) (end 187.96 74.562357) (width 0.2) (layer "F.Cu") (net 9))
 (segment (start 182.891752 118.151752) (end 177.812856 118.151752) (width 0.2) (layer "F.Cu") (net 9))
 (segment (start 174.5625 116.226396) (end 174.5625 114.168186) (width 0.2) (layer "F.Cu") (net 9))
 (segment (start 177.405056 80.037301) (end 186.322357 71.12) (width 0.2) (layer "F.Cu") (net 10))
 (segment (start 170.18 83.82) (end 173.622357 83.82) (width 0.2) (layer "F.Cu") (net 10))
 (segment (start 186.322357 71.12) (end 187.96 71.12) (width 0.2) (layer "F.Cu") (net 10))
 (segment (start 173.622357 83.82) (end 177.405056 80.037301) (width 0.2) (layer "F.Cu") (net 10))
 (via (at 170.18 83.82) (size 0.6) (drill 0.3) (layers "F.Cu" "B.Cu") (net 10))
 (segment (start 187.96 119.38) (end 189.1 118.24) (width 0.2) (layer "B.Cu") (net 10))
 (segment (start 189.1 118.24) (end 186.254315 118.24) (width 0.2) (layer "B.Cu") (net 10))
 (segment (start 186.254315 118.24) (end 170.18 102.165685) (width 0.2) (layer "B.Cu") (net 10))
 (segment (start 170.18 102.165685) (end 170.18 83.82) (width 0.2) (layer "B.Cu") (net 10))
 (segment (start 177.405056 74.957301) (end 178.5372 74.957301) (width 0.2) (layer "B.Cu") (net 14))
 (segment (start 190.5 104.14) (end 187.96 106.68) (width 0.2) (layer "B.Cu") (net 14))
 (segment (start 190.5 86.920101) (end 190.5 104.14) (width 0.2) (layer "B.Cu") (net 14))
 (segment (start 177.405056 68.974944) (end 187.96 58.42) (width 0.2) (layer "B.Cu") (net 14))
 (segment (start 177.405056 74.957301) (end 177.405056 68.974944) (width 0.2) (layer "B.Cu") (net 14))
 (segment (start 178.5372 74.957301) (end 190.5 86.920101) (width 0.2) (layer "B.Cu") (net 14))
 (segment (start 185.42 53.34) (end 187.96 53.34) (width 0.2) (layer "F.Cu") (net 3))
 (segment (start 177.8 66.04) (end 182.88 60.96) (width 0.2) (layer "F.Cu") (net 3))
 (segment (start 182.88 55.88) (end 185.42 53.34) (width 0.2) (layer "F.Cu") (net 3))
 (segment (start 182.88 60.96) (end 182.88 55.88) (width 0.2) (layer "F.Cu") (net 3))
 (segment (start 187.96 45.72) (end 184.79 45.72) (width 0.2) (layer "F.Cu") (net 21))
 (segment (start 184.79 45.72) (end 179.71 50.8) (width 0.2) (layer "F.Cu") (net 21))
 (segment (start 182.25 40.64) (end 179.71 43.18) (width 0.2) (layer "F.Cu") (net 18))
 (segment (start 187.96 40.64) (end 182.25 40.64) (width 0.2) (layer "F.Cu") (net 18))
 (segment (start 180.34 114.3) (end 177.8 116.84) (width 0.2) (layer "F.Cu") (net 4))
 (segment (start 187.96 101.6) (end 187.96 103.597817) (width 0.2) (layer "F.Cu") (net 4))
 (segment (start 180.34 111.217817) (end 180.34 114.3) (width 0.2) (layer "F.Cu") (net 4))
 (segment (start 187.96 103.597817) (end 180.34 111.217817) (width 0.2) (layer "F.Cu") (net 4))
 (segment (start 180.34 101.6) (end 187.96 93.98) (width 0.2) (layer "F.Cu") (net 7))
 (segment (start 179.71 101.6) (end 180.34 101.6) (width 0.2) (layer "F.Cu") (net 7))
 (segment (start 184.79 88.9) (end 179.71 93.98) (width 0.2) (layer "F.Cu") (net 8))
 (segment (start 187.96 88.9) (end 184.79 88.9) (width 0.2) (layer "F.Cu") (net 8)))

